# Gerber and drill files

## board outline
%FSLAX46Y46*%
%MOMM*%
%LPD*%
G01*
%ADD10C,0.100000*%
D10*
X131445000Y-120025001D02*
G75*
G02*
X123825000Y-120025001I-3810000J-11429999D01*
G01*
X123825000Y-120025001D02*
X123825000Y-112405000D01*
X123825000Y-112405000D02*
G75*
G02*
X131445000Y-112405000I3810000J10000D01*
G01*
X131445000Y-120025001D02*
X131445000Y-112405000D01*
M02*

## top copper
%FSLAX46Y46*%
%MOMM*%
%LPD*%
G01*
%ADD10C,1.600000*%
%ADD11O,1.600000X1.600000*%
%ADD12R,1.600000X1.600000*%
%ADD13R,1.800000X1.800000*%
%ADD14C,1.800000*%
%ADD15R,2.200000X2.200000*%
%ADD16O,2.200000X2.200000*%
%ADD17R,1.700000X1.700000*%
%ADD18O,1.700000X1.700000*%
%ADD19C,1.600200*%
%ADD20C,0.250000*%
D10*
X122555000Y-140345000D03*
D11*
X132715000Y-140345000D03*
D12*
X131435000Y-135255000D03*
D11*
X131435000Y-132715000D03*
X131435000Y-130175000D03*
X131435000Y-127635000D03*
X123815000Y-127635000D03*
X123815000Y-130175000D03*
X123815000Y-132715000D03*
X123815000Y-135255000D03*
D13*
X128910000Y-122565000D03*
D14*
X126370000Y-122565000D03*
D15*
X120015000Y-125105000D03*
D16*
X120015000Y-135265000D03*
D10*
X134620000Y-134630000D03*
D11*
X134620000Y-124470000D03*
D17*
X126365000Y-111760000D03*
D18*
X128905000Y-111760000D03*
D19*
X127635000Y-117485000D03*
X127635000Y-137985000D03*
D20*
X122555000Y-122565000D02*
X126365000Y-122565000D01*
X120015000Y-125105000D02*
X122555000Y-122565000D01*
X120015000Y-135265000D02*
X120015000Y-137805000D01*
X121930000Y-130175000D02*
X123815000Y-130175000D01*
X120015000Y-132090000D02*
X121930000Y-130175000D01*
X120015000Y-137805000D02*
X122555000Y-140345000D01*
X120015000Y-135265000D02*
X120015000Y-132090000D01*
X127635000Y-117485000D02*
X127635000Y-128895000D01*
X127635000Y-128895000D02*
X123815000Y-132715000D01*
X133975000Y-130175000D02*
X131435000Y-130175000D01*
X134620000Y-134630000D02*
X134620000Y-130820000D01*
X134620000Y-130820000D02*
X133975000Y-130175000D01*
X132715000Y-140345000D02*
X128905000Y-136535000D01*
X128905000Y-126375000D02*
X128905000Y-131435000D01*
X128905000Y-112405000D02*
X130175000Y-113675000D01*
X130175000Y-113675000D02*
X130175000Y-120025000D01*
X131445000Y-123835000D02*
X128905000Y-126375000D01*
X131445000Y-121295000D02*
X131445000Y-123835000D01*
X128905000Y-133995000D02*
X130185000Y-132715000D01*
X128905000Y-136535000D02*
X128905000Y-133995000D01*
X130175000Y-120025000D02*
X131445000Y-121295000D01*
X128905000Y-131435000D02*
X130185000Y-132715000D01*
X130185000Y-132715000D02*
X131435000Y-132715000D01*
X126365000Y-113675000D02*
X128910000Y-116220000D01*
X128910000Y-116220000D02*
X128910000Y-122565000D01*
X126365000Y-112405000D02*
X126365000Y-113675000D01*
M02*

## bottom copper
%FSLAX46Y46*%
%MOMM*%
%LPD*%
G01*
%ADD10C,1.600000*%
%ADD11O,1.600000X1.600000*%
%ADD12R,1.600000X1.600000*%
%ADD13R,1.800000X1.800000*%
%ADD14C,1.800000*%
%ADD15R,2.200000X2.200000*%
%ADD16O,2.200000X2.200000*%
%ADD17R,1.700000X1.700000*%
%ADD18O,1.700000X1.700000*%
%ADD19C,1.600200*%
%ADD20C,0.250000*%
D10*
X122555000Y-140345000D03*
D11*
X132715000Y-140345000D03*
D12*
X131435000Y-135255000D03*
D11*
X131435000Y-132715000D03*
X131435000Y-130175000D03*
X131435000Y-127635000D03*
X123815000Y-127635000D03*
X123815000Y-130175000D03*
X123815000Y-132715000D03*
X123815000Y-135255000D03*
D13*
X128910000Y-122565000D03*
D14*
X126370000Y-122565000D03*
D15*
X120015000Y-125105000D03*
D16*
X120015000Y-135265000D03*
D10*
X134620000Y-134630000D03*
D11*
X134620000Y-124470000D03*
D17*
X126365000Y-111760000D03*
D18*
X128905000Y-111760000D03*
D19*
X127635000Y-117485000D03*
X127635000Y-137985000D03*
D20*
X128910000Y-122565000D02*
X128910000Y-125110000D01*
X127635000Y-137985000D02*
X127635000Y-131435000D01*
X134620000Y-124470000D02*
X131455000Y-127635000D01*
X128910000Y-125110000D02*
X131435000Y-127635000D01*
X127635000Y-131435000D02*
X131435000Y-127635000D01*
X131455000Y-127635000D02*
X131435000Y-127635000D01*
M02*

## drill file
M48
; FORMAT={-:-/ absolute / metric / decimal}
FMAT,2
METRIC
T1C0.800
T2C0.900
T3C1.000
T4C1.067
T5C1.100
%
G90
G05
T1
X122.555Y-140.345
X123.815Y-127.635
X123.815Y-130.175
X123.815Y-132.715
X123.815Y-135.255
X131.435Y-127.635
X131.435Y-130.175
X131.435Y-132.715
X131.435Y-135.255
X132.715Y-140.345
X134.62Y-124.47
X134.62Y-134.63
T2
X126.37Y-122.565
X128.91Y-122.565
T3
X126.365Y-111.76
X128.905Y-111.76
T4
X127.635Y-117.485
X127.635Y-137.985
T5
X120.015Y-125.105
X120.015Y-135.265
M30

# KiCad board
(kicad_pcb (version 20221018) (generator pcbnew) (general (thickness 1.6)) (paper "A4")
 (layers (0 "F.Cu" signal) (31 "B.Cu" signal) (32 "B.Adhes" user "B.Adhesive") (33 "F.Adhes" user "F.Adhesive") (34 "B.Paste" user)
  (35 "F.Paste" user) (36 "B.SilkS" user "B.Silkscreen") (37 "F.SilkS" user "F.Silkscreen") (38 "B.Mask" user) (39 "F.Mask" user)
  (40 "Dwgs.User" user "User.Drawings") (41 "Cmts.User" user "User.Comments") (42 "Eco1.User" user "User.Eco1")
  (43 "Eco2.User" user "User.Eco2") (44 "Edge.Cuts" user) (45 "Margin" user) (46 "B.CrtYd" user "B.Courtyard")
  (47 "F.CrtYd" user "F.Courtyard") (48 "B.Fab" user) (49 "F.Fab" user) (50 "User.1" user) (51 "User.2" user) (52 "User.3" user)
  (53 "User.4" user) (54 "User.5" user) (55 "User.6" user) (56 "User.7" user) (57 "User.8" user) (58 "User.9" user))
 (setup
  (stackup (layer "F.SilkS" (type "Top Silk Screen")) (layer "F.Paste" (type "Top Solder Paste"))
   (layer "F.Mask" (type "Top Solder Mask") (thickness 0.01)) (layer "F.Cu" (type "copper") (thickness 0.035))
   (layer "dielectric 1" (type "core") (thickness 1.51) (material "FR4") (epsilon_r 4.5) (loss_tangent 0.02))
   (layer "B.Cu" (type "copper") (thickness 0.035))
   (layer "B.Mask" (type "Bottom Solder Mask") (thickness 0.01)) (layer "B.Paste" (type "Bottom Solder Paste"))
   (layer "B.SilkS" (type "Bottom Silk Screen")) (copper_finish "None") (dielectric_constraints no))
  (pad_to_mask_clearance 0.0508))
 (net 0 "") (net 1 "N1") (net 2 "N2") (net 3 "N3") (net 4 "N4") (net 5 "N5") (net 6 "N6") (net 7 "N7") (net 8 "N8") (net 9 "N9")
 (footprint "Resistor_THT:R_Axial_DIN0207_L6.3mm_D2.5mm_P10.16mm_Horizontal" (layer "F.Cu") (at 122.555 140.345)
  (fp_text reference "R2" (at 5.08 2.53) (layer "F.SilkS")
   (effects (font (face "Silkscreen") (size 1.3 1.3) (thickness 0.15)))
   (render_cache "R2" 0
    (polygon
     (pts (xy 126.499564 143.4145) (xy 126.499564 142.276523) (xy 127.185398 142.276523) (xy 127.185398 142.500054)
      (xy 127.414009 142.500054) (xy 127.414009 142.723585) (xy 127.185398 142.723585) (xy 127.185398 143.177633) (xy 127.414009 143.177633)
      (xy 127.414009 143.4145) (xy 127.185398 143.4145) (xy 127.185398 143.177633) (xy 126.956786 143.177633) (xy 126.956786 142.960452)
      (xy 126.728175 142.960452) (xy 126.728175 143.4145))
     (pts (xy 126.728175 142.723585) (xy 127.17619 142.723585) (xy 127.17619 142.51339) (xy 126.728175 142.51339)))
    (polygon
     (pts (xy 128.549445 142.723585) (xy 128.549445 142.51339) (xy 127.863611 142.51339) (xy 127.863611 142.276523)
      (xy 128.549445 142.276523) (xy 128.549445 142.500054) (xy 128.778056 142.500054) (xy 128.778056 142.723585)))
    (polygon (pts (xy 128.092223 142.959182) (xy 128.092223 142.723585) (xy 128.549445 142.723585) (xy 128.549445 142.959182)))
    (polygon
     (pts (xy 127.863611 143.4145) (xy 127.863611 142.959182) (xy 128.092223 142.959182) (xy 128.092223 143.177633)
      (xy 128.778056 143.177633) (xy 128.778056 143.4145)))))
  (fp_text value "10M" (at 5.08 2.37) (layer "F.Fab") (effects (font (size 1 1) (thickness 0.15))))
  (pad "1" thru_hole circle (at 0 0) (size 1.6 1.6) (drill 0.8) (layers "*.Cu" "*.Mask") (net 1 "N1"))
  (pad "2" thru_hole oval (at 10.16 0) (size 1.6 1.6) (drill 0.8) (layers "*.Cu" "*.Mask") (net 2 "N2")))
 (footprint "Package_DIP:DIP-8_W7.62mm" (layer "F.Cu") (at 131.435 135.255 180)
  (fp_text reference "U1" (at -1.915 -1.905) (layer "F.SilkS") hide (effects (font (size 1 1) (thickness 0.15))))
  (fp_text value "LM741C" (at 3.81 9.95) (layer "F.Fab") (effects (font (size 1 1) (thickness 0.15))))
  (pad "1" thru_hole rect (at 0 0 180) (size 1.6 1.6) (drill 0.8) (layers "*.Cu" "*.Mask") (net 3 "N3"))
  (pad "2" thru_hole oval (at 0 2.54 180) (size 1.6 1.6) (drill 0.8) (layers "*.Cu" "*.Mask") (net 2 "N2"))
  (pad "3" thru_hole oval (at 0 5.08 180) (size 1.6 1.6) (drill 0.8) (layers "*.Cu" "*.Mask") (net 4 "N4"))
  (pad "4" thru_hole oval (at 0 7.62 180) (size 1.6 1.6) (drill 0.8) (layers "*.Cu" "*.Mask") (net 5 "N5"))
  (pad "5" thru_hole oval (at 7.62 7.62 180) (size 1.6 1.6) (drill 0.8) (layers "*.Cu" "*.Mask") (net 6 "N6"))
  (pad "6" thru_hole oval (at 7.62 5.08 180) (size 1.6 1.6) (drill 0.8) (layers "*.Cu" "*.Mask") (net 1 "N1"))
  (pad "7" thru_hole oval (at 7.62 2.54 180) (size 1.6 1.6) (drill 0.8) (layers "*.Cu" "*.Mask") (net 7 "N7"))
  (pad "8" thru_hole oval (at 7.62 0 180) (size 1.6 1.6) (drill 0.8) (layers "*.Cu" "*.Mask") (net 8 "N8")))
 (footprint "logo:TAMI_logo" (layer "F.Cu") (at 127.508 114.3)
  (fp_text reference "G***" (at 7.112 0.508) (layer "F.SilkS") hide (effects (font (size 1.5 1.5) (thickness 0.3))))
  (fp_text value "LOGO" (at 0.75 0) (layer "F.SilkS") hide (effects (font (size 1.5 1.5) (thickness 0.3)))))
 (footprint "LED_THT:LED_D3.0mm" (layer "F.Cu") (at 128.91 122.565 180)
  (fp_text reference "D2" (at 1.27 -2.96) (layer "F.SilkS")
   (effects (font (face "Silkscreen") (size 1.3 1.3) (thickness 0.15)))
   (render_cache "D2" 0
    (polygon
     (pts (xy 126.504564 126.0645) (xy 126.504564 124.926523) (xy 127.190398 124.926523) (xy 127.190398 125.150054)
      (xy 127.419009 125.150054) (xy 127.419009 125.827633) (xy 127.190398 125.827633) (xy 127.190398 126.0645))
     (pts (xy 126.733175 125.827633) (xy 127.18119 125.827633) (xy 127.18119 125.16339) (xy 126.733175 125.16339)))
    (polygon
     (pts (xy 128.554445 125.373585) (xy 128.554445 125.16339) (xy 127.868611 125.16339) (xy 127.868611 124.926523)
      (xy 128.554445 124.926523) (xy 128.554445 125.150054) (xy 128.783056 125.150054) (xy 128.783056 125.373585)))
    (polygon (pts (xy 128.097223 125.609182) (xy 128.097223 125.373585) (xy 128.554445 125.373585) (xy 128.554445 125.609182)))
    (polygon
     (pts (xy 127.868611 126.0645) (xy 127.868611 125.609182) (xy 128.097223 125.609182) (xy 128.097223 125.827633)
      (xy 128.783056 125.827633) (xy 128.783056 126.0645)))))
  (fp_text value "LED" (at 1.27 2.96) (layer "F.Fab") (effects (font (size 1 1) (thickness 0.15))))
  (pad "1" thru_hole rect (at 0 0 180) (size 1.8 1.8) (drill 0.9) (layers "*.Cu" "*.Mask") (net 5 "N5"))
  (pad "2" thru_hole circle (at 2.54 0 180) (size 1.8 1.8) (drill 0.9) (layers "*.Cu" "*.Mask") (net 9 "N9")))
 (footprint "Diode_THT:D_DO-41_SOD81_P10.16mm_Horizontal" (layer "F.Cu") (at 120.015 125.105 -90)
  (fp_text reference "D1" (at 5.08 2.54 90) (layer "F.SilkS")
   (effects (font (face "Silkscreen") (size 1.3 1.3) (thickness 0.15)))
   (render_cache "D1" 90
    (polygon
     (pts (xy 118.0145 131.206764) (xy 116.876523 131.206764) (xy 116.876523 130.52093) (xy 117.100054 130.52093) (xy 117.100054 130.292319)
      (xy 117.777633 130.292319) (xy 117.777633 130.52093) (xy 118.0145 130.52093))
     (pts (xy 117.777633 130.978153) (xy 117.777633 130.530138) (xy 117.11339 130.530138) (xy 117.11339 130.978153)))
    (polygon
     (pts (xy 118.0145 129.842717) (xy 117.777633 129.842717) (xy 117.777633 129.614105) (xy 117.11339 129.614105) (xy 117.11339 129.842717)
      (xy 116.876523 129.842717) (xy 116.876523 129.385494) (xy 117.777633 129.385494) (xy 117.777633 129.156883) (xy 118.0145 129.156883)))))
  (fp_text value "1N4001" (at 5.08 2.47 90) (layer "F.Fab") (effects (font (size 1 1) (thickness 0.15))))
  (pad "1" thru_hole rect (at 0 0 270) (size 2.2 2.2) (drill 1.1) (layers "*.Cu" "*.Mask") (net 9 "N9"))
  (pad "2" thru_hole oval (at 10.16 0 270) (size 2.2 2.2) (drill 1.1) (layers "*.Cu" "*.Mask") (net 1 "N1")))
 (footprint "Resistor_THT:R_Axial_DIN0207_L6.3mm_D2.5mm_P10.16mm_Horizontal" (layer "F.Cu") (at 134.62 134.63 90)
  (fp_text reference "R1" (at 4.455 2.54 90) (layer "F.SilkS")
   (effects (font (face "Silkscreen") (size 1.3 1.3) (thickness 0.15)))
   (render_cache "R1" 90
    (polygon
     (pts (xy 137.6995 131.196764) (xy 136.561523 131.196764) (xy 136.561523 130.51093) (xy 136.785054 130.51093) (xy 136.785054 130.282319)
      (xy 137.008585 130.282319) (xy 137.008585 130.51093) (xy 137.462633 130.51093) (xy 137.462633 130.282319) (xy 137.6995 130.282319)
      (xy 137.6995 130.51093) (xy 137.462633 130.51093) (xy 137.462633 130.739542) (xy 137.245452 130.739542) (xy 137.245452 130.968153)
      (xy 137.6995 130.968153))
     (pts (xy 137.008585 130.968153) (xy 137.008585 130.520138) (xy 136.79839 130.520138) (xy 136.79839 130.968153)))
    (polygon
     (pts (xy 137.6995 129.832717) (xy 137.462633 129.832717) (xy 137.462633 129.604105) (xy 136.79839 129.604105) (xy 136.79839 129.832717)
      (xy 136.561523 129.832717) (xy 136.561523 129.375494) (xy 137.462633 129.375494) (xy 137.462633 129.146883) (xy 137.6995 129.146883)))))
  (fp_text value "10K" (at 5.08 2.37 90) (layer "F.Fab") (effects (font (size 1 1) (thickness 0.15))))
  (pad "1" thru_hole circle (at 0 0 90) (size 1.6 1.6) (drill 0.8) (layers "*.Cu" "*.Mask") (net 4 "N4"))
  (pad "2" thru_hole oval (at 10.16 0 90) (size 1.6 1.6) (drill 0.8) (layers "*.Cu" "*.Mask") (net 5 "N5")))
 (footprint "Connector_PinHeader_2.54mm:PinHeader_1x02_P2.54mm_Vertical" (layer "B.Cu") (at 126.365 111.76 -90)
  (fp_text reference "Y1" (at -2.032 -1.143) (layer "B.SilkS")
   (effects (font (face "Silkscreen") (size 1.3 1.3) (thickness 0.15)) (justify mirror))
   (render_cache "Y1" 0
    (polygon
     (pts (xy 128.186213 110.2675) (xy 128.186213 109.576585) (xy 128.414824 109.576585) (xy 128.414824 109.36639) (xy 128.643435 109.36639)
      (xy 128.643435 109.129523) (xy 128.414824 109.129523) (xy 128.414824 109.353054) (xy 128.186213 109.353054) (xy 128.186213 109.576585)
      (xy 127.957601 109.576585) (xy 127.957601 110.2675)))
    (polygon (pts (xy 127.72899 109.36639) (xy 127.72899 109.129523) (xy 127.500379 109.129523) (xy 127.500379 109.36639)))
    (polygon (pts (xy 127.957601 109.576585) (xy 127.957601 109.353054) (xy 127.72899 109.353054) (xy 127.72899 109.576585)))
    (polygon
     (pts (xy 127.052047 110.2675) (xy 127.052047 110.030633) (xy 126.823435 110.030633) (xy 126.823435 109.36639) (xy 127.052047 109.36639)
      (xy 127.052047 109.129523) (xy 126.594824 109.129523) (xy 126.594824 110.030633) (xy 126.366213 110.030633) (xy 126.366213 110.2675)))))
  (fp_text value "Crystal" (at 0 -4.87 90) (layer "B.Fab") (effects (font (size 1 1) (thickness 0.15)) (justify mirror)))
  (pad "1" thru_hole rect (at 0 0 270) (size 1.7 1.7) (drill 1) (layers "*.Cu" "*.Mask") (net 5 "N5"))
  (pad "2" thru_hole oval (at 0 -2.54 270) (size 1.7 1.7) (drill 1) (layers "*.Cu" "*.Mask") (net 2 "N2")))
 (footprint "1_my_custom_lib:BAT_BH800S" (layer "B.Cu") (at 127.635 131.485)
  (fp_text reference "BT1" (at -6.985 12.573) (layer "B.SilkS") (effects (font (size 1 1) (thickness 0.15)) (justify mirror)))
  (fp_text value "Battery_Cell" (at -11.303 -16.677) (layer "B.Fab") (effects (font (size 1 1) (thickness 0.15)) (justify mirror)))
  (pad "1" thru_hole circle (at 0 -14) (size 1.6002 1.6002) (drill 1.0668) (layers "*.Cu" "*.Mask") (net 7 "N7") (solder_mask_margin 0.102))
  (pad "2" thru_hole circle (at 0 6.5) (size 1.6002 1.6002) (drill 1.0668) (layers "*.Cu" "*.Mask") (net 5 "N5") (solder_mask_margin 0.102)))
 (gr_arc (start 131.445 120.025001) (mid 127.635 143.503277) (end 123.825 120.025001) (stroke (width 0.1) (type default))
  (layer "Edge.Cuts"))
 (gr_line (start 123.825 120.025001) (end 123.825 112.405) (stroke (width 0.1) (type default)) (layer "Edge.Cuts"))
 (gr_arc (start 123.825 112.405) (mid 127.635 108.584987) (end 131.445 112.405) (stroke (width 0.1) (type default)) (layer "Edge.Cuts"))
 (gr_line (start 131.445 120.025001) (end 131.445 112.405) (stroke (width 0.1) (type default)) (layer "Edge.Cuts"))
 (segment (start 122.555 122.565) (end 126.365 122.565) (width 0.25) (layer "F.Cu") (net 9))
 (segment (start 120.015 125.105) (end 122.555 122.565) (width 0.25) (layer "F.Cu") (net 9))
 (segment (start 120.015 135.265) (end 120.015 137.805) (width 0.25) (layer "F.Cu") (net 1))
 (segment (start 121.93 130.175) (end 123.815 130.175) (width 0.25) (layer "F.Cu") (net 1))
 (segment (start 120.015 132.09) (end 121.93 130.175) (width 0.25) (layer "F.Cu") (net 1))
 (segment (start 120.015 137.805) (end 122.555 140.345) (width 0.25) (layer "F.Cu") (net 1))
 (segment (start 120.015 135.265) (end 120.015 132.09) (width 0.25) (layer "F.Cu") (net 1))
 (segment (start 127.635 117.485) (end 127.635 128.895) (width 0.25) (layer "F.Cu") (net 7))
 (segment (start 127.635 128.895) (end 123.815 132.715) (width 0.25) (layer "F.Cu") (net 7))
 (segment (start 133.975 130.175) (end 131.435 130.175) (width 0.25) (layer "F.Cu") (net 4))
 (segment (start 134.62 134.63) (end 134.62 130.82) (width 0.25) (layer "F.Cu") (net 4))
 (segment (start 134.62 130.82) (end 133.975 130.175) (width 0.25) (layer "F.Cu") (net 4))
 (segment (start 132.715 140.345) (end 128.905 136.535) (width 0.25) (layer "F.Cu") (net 2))
 (segment (start 128.905 126.375) (end 128.905 131.435) (width 0.25) (layer "F.Cu") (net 2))
 (segment (start 128.905 112.405) (end 130.175 113.675) (width 0.25) (layer "F.Cu") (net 2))
 (segment (start 130.175 113.675) (end 130.175 120.025) (width 0.25) (layer "F.Cu") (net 2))
 (segment (start 131.445 123.835) (end 128.905 126.375) (width 0.25) (layer "F.Cu") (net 2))
 (segment (start 131.445 121.295) (end 131.445 123.835) (width 0.25) (layer "F.Cu") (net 2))
 (segment (start 128.905 133.995) (end 130.185 132.715) (width 0.25) (layer "F.Cu") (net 2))
 (segment (start 128.905 136.535) (end 128.905 133.995) (width 0.25) (layer "F.Cu") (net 2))
 (segment (start 130.175 120.025) (end 131.445 121.295) (width 0.25) (layer "F.Cu") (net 2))
 (segment (start 128.905 131.435) (end 130.185 132.715) (width 0.25) (layer "F.Cu") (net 2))
 (segment (start 130.185 132.715) (end 131.435 132.715) (width 0.25) (layer "F.Cu") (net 2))
 (segment (start 126.365 113.675) (end 128.91 116.22) (width 0.25) (layer "F.Cu") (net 5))
 (segment (start 128.91 116.22) (end 128.91 122.565) (width 0.25) (layer "F.Cu") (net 5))
 (segment (start 126.365 112.405) (end 126.365 113.675) (width 0.25) (layer "F.Cu") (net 5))
 (segment (start 128.91 122.565) (end 128.91 125.11) (width 0.25) (layer "B.Cu") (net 5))
 (segment (start 127.635 137.985) (end 127.635 131.435) (width 0.25) (layer "B.Cu") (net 5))
 (segment (start 134.62 124.47) (end 131.455 127.635) (width 0.25) (layer "B.Cu") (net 5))
 (segment (start 128.91 125.11) (end 131.435 127.635) (width 0.25) (layer "B.Cu") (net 5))
 (segment (start 127.635 131.435) (end 131.435 127.635) (width 0.25) (layer "B.Cu") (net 5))
 (segment (start 131.455 127.635) (end 131.435 127.635) (width 0.25) (layer "B.Cu") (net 5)))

